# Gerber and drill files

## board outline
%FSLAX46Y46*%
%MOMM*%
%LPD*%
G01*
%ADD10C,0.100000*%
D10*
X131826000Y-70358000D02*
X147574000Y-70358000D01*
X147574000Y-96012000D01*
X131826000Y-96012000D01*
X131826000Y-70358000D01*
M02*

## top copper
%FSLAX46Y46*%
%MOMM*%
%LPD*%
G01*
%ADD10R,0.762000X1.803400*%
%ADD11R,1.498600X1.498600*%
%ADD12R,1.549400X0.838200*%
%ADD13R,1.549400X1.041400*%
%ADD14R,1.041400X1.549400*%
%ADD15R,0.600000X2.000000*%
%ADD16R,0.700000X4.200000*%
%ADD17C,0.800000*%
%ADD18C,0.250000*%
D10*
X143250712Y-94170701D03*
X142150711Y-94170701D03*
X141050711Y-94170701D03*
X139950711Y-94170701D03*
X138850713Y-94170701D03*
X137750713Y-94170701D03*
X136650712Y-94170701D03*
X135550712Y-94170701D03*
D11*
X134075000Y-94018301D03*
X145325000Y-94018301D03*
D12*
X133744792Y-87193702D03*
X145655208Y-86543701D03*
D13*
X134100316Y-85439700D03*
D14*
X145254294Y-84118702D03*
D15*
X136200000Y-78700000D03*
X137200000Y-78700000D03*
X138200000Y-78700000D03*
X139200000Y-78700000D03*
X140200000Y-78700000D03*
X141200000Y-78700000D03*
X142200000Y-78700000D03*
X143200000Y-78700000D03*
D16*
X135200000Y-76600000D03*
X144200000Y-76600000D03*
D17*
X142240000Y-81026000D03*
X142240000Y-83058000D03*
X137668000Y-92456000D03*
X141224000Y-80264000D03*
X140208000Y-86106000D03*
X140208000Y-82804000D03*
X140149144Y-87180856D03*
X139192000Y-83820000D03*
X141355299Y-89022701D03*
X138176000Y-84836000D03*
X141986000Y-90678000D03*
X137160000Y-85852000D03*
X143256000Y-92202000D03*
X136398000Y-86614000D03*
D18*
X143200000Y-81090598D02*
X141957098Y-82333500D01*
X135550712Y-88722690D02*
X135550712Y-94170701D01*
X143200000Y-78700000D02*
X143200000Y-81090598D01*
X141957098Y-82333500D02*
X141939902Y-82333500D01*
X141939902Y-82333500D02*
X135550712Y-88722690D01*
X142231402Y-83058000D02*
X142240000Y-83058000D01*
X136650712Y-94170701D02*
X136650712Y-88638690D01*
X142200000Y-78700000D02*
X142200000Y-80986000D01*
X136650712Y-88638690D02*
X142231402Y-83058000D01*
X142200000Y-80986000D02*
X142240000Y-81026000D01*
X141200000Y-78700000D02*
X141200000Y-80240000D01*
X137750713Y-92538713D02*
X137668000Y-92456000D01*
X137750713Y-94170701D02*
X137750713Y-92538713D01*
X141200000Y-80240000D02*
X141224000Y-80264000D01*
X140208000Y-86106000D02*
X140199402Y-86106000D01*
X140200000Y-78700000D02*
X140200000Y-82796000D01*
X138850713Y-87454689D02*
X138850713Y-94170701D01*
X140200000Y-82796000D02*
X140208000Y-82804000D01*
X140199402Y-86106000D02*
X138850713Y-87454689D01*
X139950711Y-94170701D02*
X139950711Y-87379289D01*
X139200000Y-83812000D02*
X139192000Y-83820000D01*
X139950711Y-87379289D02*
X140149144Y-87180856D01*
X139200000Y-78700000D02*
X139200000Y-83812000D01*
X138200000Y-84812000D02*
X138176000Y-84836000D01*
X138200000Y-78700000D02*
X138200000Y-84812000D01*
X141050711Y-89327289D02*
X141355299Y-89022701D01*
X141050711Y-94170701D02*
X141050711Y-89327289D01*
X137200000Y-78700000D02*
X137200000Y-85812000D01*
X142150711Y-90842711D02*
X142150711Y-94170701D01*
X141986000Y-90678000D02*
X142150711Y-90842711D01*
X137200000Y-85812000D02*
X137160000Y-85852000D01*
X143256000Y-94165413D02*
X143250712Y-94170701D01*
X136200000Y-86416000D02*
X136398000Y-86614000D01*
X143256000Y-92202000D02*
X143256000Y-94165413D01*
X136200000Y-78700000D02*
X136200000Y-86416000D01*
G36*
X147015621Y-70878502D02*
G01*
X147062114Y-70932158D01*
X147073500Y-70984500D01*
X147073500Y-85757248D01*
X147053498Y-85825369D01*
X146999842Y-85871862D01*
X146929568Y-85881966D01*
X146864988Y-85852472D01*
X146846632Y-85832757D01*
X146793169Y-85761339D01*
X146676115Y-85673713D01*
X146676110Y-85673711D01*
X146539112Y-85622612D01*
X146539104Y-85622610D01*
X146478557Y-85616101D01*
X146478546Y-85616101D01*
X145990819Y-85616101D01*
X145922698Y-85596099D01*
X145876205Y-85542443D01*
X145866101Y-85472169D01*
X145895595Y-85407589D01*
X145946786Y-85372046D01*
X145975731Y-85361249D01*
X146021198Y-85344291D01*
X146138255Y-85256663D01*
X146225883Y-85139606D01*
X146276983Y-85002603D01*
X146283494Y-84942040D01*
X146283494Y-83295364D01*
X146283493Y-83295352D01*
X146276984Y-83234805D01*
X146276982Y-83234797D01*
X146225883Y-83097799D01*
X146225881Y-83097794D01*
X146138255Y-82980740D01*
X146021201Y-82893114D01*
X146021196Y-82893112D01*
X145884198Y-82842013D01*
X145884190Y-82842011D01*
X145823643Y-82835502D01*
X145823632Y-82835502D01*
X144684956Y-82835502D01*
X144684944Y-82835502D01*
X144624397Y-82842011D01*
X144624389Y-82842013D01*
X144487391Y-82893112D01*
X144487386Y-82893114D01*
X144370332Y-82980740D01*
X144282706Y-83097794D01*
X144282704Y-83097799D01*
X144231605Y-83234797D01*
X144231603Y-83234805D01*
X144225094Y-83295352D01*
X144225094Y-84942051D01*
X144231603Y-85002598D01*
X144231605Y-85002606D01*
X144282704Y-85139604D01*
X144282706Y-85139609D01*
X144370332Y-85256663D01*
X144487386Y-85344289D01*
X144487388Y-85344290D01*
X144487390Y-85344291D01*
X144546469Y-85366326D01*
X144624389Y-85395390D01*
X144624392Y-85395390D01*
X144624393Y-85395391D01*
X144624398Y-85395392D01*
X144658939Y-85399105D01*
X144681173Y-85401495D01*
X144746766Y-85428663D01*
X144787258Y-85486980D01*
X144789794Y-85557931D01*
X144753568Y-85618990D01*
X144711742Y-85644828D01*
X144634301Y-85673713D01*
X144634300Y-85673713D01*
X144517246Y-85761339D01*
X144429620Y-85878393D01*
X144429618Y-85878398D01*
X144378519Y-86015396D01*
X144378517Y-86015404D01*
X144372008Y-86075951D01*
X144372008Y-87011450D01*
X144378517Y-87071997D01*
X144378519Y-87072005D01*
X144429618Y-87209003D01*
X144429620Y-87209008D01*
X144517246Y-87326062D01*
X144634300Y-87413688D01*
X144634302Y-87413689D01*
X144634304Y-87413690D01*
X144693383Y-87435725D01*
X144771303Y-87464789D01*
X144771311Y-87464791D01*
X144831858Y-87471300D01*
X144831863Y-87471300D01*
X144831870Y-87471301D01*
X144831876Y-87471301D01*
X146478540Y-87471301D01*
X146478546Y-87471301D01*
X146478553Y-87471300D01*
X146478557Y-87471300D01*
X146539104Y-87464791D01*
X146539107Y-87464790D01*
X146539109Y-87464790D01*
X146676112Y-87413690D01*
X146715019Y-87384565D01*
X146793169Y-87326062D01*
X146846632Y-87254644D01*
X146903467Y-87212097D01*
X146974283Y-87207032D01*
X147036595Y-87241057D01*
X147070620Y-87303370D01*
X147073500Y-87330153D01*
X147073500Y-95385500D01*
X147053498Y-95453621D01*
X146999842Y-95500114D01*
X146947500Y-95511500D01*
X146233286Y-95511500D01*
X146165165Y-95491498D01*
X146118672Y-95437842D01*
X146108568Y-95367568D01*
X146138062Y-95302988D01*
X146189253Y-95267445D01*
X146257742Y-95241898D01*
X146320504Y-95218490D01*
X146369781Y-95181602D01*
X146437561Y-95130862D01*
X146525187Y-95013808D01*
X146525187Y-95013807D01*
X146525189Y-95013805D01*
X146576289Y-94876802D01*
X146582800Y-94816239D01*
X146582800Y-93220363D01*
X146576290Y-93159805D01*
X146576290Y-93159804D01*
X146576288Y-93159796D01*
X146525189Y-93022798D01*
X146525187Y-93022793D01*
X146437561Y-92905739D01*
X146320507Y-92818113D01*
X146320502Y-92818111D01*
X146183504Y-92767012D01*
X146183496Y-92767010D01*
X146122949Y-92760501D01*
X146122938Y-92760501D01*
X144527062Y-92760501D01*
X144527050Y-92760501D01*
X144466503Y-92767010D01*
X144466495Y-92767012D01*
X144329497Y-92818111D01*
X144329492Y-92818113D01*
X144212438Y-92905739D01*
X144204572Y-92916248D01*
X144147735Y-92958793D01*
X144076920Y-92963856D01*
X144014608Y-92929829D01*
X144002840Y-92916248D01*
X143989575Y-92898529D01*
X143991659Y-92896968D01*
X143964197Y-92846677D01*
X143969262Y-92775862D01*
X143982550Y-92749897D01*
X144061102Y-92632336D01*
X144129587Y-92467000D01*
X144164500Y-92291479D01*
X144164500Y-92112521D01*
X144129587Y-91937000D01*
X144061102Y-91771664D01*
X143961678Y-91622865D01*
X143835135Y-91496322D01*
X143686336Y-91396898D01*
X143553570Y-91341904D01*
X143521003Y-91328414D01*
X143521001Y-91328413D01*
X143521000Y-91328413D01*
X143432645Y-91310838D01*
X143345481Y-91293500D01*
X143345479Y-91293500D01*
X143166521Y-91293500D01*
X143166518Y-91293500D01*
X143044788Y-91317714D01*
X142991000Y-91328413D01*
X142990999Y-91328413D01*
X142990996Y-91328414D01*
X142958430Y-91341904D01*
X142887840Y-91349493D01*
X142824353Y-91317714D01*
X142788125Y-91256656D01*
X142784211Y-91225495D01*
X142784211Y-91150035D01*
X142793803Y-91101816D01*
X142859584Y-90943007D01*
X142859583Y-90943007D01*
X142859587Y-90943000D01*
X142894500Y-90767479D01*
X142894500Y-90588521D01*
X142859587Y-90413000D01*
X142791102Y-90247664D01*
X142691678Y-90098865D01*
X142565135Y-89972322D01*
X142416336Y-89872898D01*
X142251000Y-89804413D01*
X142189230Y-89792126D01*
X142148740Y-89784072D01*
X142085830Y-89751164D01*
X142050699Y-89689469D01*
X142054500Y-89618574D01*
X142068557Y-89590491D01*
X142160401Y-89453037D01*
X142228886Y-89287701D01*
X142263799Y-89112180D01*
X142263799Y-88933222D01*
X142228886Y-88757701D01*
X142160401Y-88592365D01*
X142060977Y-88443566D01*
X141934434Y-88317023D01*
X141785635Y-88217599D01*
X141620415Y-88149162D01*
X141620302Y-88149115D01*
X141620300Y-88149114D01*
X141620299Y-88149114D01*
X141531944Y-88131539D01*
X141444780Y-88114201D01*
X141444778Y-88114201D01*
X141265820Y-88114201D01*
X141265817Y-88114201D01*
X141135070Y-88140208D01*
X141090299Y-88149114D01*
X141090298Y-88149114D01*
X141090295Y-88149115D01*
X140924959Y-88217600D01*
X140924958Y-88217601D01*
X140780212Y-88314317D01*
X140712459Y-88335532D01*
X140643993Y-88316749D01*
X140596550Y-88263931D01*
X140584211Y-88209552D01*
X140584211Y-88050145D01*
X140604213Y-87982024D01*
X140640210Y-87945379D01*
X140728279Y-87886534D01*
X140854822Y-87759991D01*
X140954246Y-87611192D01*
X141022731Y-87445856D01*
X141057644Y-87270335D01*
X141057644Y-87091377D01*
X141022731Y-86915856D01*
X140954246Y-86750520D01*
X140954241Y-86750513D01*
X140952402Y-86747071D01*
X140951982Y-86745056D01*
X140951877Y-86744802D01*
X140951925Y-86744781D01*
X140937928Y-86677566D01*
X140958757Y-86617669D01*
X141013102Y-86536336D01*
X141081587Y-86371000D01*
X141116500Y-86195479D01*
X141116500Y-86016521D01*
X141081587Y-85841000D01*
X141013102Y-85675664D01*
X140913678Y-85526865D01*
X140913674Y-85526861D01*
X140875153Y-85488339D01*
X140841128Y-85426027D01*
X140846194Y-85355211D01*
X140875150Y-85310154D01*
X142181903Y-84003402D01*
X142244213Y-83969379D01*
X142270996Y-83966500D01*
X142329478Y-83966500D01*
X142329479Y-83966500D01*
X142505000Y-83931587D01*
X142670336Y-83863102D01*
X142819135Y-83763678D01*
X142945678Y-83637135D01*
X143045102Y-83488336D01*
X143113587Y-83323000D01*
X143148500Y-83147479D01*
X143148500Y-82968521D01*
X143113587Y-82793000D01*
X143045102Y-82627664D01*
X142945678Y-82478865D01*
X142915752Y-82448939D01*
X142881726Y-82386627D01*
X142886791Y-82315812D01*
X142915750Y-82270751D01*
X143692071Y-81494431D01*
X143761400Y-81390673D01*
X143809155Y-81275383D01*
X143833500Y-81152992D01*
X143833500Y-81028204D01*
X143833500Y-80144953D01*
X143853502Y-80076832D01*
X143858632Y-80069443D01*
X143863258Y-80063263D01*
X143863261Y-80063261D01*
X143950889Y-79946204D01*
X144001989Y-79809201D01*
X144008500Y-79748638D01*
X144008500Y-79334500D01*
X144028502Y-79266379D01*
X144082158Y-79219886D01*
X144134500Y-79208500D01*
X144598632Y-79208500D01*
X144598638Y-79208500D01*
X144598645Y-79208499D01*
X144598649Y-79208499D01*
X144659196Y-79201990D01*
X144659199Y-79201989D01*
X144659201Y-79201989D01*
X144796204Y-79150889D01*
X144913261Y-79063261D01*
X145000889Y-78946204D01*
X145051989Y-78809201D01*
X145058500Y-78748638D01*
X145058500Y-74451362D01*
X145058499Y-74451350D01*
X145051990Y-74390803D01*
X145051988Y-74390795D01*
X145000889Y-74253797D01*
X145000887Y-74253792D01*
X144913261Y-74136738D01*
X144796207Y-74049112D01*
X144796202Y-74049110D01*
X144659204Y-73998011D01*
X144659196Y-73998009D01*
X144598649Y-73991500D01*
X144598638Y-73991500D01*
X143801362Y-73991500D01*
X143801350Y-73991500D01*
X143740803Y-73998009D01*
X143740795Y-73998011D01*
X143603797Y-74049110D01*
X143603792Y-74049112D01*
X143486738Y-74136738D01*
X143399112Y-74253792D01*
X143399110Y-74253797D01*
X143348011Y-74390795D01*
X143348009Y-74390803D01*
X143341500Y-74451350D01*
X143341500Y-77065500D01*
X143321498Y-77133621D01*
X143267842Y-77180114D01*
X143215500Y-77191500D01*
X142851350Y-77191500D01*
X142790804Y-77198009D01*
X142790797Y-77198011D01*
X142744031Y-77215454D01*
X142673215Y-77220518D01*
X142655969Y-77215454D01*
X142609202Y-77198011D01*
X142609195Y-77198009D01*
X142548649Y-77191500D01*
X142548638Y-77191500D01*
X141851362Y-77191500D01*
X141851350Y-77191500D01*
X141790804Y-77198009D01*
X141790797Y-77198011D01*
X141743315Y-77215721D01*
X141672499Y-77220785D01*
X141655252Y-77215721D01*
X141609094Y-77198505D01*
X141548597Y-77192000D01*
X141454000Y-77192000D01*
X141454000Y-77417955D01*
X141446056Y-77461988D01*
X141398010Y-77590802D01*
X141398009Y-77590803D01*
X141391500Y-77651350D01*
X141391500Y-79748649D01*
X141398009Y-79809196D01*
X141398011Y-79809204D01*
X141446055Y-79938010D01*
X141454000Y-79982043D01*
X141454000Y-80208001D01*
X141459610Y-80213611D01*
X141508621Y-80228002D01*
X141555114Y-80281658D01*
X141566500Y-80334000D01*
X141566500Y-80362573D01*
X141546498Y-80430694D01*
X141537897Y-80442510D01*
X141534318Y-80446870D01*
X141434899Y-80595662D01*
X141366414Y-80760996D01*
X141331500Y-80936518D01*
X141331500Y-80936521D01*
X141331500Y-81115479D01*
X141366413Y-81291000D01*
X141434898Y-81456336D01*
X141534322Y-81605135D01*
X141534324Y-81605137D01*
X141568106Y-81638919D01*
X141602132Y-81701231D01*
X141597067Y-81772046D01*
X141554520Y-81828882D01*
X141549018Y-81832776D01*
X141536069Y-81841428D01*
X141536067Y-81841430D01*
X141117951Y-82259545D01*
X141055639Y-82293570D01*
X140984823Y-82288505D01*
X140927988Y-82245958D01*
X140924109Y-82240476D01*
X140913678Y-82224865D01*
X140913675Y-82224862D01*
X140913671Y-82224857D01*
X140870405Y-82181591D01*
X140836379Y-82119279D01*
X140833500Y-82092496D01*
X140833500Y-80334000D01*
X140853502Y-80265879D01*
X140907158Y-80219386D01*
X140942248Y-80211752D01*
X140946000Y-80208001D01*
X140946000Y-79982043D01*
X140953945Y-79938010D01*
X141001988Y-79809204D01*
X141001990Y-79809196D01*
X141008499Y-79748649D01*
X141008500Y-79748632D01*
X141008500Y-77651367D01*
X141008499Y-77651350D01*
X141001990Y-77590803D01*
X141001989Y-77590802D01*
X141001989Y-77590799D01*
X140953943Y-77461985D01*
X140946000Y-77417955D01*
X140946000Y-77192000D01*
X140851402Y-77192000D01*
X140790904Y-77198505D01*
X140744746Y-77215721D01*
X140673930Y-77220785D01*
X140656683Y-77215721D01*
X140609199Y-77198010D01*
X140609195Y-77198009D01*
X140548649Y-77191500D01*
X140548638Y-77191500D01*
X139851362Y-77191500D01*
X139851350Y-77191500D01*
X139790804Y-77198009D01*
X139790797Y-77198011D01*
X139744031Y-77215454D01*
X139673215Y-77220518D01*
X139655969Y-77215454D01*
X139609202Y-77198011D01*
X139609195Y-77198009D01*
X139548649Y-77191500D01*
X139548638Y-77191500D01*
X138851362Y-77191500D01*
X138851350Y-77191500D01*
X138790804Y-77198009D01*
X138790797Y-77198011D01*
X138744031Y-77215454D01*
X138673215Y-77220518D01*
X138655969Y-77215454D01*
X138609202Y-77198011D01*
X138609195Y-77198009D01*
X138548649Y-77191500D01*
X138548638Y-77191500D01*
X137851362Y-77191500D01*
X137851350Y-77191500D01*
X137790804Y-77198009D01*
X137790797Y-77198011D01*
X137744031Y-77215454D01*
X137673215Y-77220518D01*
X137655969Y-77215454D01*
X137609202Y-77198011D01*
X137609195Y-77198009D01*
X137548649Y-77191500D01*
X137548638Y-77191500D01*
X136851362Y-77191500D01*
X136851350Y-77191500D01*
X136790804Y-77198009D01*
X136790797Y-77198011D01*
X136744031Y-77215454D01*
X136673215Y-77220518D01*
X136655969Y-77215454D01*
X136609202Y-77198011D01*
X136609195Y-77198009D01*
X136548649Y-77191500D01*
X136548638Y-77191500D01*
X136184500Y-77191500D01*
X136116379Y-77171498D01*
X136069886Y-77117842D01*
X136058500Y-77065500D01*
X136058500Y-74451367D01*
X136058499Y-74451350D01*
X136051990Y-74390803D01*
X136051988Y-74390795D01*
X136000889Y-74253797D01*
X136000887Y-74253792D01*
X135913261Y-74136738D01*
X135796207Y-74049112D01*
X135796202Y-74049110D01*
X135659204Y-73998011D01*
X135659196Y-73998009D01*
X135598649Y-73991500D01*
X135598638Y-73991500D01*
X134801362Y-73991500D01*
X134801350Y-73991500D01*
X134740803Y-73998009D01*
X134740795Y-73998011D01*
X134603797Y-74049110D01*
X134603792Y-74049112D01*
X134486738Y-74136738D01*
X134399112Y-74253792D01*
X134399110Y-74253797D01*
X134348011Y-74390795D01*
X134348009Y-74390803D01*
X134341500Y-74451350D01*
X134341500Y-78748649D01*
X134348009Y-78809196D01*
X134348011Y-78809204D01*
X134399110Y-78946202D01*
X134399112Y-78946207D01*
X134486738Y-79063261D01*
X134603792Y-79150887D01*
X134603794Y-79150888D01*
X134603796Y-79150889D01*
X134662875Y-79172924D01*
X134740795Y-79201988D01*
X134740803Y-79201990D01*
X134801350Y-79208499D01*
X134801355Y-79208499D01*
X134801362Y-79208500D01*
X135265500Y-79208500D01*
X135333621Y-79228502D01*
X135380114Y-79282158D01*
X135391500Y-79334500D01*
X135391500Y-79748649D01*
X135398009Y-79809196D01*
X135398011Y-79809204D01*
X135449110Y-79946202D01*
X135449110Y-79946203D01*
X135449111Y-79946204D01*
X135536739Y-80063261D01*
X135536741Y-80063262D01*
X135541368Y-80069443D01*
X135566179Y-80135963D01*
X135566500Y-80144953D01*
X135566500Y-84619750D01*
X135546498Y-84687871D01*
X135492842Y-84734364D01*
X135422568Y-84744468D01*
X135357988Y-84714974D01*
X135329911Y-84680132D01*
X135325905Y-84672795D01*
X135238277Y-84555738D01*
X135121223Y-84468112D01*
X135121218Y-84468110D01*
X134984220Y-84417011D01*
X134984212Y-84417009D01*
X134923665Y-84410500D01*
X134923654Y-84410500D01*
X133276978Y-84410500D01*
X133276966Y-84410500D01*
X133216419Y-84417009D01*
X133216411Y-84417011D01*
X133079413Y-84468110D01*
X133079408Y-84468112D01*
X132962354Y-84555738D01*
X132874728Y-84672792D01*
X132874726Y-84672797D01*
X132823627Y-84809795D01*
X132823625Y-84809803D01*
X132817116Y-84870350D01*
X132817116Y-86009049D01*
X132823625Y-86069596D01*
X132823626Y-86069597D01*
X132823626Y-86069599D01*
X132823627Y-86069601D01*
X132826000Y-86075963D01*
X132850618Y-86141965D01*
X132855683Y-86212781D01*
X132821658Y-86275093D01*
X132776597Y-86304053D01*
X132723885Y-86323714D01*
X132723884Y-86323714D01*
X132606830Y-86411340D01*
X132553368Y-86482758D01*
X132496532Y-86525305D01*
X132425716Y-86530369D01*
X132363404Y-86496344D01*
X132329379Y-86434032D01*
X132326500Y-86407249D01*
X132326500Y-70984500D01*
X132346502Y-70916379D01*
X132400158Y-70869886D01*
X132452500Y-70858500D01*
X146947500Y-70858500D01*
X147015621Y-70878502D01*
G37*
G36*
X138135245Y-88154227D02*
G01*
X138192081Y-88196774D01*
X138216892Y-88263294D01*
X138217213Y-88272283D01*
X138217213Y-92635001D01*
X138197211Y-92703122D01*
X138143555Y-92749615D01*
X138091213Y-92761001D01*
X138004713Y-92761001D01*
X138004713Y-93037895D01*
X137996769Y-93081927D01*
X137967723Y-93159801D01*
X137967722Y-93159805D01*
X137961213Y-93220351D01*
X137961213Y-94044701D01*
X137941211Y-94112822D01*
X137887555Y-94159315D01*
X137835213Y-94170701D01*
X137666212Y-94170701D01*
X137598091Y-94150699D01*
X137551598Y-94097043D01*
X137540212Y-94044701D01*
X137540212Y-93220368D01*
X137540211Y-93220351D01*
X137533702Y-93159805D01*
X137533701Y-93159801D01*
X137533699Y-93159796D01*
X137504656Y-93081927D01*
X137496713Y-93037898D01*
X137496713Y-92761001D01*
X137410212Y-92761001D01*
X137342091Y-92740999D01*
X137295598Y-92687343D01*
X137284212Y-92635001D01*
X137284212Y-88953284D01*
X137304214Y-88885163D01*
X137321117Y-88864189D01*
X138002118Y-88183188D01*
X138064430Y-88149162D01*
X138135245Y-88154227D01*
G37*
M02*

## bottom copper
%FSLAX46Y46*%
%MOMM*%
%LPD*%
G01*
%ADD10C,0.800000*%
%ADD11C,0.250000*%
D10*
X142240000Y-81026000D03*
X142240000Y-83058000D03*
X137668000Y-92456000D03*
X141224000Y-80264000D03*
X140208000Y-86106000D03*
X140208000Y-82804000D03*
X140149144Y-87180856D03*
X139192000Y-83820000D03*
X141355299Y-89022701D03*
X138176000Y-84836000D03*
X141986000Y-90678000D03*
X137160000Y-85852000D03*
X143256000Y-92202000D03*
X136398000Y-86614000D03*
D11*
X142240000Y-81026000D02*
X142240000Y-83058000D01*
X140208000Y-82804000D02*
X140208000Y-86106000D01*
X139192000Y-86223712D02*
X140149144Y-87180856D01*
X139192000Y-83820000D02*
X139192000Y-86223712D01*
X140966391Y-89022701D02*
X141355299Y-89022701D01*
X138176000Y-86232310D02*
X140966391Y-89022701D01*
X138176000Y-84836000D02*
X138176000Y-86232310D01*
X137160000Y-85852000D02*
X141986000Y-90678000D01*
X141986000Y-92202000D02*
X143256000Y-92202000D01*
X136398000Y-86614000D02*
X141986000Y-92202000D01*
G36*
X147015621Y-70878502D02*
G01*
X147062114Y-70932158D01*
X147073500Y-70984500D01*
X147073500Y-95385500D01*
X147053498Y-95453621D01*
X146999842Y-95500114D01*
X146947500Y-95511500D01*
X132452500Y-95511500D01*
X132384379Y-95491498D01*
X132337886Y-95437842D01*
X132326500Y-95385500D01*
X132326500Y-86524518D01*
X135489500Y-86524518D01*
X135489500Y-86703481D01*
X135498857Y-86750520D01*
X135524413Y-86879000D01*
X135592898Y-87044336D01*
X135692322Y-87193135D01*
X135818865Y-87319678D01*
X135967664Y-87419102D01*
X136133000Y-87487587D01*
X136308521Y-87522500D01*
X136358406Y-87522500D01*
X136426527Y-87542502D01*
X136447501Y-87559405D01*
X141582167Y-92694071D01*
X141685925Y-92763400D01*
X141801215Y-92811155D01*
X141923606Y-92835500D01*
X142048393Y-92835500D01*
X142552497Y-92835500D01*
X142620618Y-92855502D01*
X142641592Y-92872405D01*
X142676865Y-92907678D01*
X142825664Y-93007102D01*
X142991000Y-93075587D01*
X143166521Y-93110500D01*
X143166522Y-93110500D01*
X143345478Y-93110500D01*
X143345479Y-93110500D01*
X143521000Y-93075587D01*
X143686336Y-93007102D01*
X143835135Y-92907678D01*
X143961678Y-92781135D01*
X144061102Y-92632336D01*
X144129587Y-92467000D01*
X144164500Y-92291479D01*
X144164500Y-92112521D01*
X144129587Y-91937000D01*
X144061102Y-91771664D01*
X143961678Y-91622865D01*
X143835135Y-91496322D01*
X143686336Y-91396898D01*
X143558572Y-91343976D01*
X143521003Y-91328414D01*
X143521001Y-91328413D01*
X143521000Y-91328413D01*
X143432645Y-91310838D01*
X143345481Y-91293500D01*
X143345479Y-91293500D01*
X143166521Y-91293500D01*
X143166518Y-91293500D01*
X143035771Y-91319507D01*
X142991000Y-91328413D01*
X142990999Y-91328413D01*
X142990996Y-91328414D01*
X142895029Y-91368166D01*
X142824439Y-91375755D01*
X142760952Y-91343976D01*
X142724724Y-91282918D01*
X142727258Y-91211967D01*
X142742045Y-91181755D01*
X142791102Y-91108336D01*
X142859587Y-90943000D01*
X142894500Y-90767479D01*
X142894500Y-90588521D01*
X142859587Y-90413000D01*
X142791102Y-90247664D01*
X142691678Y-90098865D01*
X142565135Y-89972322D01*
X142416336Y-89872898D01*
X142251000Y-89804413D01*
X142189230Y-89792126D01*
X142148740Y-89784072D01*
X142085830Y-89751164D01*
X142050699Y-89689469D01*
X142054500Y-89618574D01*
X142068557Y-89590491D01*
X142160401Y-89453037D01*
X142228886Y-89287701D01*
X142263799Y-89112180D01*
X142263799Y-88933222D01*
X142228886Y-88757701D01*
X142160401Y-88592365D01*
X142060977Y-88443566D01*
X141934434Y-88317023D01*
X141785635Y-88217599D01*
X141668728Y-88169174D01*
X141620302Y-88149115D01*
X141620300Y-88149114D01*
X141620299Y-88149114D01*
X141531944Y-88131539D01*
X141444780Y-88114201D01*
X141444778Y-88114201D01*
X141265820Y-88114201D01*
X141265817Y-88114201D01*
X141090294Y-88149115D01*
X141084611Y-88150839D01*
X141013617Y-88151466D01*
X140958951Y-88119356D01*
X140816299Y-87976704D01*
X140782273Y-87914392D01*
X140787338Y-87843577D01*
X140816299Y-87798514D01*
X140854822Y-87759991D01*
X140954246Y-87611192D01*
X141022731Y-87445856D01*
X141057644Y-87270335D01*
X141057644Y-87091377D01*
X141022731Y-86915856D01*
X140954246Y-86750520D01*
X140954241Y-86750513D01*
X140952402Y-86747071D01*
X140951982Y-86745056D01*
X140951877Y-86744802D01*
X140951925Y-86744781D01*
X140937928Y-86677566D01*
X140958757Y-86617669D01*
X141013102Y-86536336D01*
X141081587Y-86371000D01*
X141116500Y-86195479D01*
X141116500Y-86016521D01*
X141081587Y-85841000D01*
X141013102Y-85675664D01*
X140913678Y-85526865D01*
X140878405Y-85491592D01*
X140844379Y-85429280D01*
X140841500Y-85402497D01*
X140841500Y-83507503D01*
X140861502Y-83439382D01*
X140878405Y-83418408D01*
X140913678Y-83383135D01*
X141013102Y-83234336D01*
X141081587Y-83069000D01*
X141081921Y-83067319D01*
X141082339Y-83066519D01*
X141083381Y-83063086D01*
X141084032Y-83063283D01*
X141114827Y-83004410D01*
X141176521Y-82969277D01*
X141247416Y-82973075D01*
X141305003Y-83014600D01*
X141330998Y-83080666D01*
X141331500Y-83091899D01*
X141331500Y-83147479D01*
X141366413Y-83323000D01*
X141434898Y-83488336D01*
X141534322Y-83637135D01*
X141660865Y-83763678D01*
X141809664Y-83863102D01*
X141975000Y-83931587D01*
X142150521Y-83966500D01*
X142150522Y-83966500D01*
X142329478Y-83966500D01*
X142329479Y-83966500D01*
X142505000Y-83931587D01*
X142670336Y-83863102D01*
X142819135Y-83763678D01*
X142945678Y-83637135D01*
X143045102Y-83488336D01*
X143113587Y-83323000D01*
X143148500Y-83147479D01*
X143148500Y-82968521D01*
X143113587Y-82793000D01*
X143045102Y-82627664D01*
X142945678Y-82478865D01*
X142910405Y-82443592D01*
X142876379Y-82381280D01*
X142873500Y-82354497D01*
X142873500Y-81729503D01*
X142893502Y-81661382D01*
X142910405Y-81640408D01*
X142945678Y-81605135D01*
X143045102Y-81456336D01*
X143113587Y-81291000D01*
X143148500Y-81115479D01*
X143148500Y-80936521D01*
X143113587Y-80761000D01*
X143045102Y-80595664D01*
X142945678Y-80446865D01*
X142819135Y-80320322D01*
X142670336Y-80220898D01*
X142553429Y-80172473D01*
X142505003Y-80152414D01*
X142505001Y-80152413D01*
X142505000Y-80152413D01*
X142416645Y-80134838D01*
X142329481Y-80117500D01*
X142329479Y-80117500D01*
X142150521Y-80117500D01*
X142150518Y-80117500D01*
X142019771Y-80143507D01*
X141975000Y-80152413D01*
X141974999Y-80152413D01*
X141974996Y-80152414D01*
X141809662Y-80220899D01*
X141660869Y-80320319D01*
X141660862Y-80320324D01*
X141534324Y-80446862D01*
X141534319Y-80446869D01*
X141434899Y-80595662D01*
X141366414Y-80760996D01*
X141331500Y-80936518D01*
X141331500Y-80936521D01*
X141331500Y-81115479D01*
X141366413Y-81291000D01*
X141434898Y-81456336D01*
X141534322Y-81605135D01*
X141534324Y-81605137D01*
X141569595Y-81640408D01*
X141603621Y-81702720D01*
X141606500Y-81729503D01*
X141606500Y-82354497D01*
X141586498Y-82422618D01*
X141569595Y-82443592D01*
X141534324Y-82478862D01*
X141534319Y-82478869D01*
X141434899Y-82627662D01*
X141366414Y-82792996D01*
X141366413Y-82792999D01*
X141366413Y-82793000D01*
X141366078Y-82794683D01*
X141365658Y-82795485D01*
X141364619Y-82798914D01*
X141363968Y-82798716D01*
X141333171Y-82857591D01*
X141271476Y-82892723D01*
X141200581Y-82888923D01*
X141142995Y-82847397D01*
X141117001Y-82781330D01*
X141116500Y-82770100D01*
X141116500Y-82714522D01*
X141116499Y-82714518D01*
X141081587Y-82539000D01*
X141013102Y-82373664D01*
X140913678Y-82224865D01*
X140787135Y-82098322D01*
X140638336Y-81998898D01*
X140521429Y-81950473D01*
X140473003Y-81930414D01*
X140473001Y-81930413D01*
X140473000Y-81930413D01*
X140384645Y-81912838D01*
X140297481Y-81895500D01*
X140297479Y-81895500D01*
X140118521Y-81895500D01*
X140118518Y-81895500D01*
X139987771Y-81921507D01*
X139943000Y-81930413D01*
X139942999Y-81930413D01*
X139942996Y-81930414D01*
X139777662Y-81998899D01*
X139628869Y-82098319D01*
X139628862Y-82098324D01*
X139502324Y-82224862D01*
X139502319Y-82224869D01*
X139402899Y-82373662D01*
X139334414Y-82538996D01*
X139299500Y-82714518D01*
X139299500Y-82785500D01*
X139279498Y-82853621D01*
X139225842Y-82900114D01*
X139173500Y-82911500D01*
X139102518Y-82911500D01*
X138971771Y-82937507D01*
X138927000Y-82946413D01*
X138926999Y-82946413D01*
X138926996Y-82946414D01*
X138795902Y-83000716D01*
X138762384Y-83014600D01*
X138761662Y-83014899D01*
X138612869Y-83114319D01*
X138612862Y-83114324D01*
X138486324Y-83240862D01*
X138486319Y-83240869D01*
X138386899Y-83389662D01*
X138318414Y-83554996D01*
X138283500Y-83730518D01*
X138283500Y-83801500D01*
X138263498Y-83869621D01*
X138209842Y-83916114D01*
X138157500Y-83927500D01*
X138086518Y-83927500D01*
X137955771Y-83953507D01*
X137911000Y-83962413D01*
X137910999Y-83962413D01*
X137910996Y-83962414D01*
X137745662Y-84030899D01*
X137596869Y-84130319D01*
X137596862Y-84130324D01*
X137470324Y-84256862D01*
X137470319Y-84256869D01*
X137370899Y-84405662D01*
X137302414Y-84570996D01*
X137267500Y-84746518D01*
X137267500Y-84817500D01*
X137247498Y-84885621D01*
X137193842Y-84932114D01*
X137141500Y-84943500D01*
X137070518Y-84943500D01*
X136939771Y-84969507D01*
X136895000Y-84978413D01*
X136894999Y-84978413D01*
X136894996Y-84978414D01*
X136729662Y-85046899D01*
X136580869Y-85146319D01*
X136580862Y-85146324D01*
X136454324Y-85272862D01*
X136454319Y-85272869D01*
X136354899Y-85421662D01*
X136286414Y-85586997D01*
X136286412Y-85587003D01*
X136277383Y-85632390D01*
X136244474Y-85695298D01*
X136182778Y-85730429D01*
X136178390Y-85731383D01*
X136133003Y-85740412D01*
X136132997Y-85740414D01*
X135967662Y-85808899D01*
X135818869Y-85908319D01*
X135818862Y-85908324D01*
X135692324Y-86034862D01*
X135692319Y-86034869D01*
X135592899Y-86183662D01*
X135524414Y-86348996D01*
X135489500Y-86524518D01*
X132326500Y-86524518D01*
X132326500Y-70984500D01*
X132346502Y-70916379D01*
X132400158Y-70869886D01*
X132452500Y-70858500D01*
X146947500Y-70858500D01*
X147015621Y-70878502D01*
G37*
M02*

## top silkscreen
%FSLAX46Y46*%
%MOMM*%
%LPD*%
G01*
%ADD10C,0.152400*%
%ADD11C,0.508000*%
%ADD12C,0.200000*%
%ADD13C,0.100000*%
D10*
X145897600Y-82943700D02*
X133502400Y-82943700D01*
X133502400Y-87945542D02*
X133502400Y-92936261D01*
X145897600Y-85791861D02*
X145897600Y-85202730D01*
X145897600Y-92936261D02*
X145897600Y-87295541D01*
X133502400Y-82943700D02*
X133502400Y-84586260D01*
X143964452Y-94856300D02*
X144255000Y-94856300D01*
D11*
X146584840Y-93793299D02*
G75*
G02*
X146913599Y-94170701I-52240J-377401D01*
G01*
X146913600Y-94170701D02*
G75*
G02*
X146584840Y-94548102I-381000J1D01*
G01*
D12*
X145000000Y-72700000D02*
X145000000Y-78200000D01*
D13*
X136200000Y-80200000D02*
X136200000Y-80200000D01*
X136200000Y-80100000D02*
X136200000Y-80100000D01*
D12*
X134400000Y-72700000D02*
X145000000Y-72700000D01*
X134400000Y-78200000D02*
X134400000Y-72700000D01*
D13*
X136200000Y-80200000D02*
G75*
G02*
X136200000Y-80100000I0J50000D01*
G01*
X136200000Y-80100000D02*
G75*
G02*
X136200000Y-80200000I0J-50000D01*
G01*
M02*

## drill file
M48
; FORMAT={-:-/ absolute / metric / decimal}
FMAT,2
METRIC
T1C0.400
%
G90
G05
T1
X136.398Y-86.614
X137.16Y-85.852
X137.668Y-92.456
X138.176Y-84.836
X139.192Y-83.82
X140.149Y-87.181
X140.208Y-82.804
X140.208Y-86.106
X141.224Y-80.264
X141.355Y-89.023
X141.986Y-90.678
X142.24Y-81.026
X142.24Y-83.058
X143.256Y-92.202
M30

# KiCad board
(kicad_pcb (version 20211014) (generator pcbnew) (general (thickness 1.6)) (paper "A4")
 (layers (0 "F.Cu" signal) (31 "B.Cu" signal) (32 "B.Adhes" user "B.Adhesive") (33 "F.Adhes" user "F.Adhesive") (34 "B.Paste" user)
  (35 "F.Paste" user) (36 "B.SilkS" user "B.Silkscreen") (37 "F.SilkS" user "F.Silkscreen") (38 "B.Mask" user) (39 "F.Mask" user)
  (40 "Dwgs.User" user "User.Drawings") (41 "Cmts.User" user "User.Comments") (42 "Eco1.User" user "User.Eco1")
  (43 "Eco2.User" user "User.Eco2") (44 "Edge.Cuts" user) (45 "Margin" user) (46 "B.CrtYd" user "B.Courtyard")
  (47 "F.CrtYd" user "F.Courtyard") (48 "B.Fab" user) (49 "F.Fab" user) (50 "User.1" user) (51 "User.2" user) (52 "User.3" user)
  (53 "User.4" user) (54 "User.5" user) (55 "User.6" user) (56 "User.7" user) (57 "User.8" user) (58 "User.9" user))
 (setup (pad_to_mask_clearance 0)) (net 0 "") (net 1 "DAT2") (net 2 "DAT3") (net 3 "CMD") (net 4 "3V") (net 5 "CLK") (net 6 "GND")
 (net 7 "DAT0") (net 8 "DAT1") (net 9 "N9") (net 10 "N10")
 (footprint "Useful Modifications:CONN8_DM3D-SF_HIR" (layer "F.Cu") (at 139.7 88.9)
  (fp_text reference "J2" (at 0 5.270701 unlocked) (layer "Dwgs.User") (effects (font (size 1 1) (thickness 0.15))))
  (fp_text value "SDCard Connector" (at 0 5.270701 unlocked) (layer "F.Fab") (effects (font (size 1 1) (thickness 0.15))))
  (fp_line (start 6.1976 -5.9563) (end -6.1976 -5.9563) (layer "F.SilkS") (width 0.1524))
  (fp_line (start -6.1976 -0.954458) (end -6.1976 4.036261) (layer "F.SilkS") (width 0.1524))
  (fp_line (start 6.1976 -3.108139) (end 6.1976 -3.69727) (layer "F.SilkS") (width 0.1524))
  (fp_line (start 6.1976 4.036261) (end 6.1976 -1.604459) (layer "F.SilkS") (width 0.1524))
  (fp_line (start -6.1976 -5.9563) (end -6.1976 -4.31374) (layer "F.SilkS") (width 0.1524))
  (fp_line (start 4.264452 5.9563) (end 4.555 5.9563) (layer "F.SilkS") (width 0.1524))
  (fp_arc (start 6.88484 4.893299) (mid 7.119884 5.020443) (end 7.2136 5.270701) (layer "F.SilkS") (width 0.508))
  (fp_arc (start 7.2136 5.270701) (mid 7.119884 5.520958) (end 6.88484 5.648102) (layer "F.SilkS") (width 0.508))
  (pad "1" smd rect (at 3.550712 5.270701) (size 0.762 1.8034) (layers "F.Cu" "F.Paste" "F.Mask") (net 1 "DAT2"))
  (pad "2" smd rect (at 2.450711 5.270701) (size 0.762 1.8034) (layers "F.Cu" "F.Paste" "F.Mask") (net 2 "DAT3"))
  (pad "3" smd rect (at 1.350711 5.270701) (size 0.762 1.8034) (layers "F.Cu" "F.Paste" "F.Mask") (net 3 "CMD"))
  (pad "4" smd rect (at 0.250711 5.270701) (size 0.762 1.8034) (layers "F.Cu" "F.Paste" "F.Mask") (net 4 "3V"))
  (pad "5" smd rect (at -0.849287 5.270701) (size 0.762 1.8034) (layers "F.Cu" "F.Paste" "F.Mask") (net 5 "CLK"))
  (pad "6" smd rect (at -1.949287 5.270701) (size 0.762 1.8034) (layers "F.Cu" "F.Paste" "F.Mask") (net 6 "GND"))
  (pad "7" smd rect (at -3.049288 5.270701) (size 0.762 1.8034) (layers "F.Cu" "F.Paste" "F.Mask") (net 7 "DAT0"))
  (pad "8" smd rect (at -4.149288 5.270701) (size 0.762 1.8034) (layers "F.Cu" "F.Paste" "F.Mask") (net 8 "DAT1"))
  (pad "9" smd rect (at -5.625 5.118301) (size 1.4986 1.4986) (layers "F.Cu" "F.Paste" "F.Mask"))
  (pad "10" smd rect (at 5.625 5.118301) (size 1.4986 1.4986) (layers "F.Cu" "F.Paste" "F.Mask"))
  (pad "11" smd rect (at -5.955208 -1.706298) (size 1.5494 0.8382) (layers "F.Cu" "F.Paste" "F.Mask"))
  (pad "12" smd rect (at 5.955208 -2.356299) (size 1.5494 0.8382) (layers "F.Cu" "F.Paste" "F.Mask"))
  (pad "13" smd rect (at -5.599684 -3.4603) (size 1.5494 1.0414) (layers "F.Cu" "F.Paste" "F.Mask"))
  (pad "14" smd rect (at 5.554294 -4.781298) (size 1.0414 1.5494) (layers "F.Cu" "F.Paste" "F.Mask")))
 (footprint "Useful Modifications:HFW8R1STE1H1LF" (layer "F.Cu") (at 139.7 76.2 180)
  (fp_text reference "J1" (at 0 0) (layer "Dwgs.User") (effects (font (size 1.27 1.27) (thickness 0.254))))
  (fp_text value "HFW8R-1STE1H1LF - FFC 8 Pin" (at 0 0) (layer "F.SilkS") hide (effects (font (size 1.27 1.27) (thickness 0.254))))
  (fp_line (start -5.3 3.5) (end -5.3 -2) (layer "F.SilkS") (width 0.2))
  (fp_line (start 3.5 -4) (end 3.5 -4) (layer "F.SilkS") (width 0.1))
  (fp_line (start 3.5 -3.9) (end 3.5 -3.9) (layer "F.SilkS") (width 0.1))
  (fp_line (start 5.3 3.5) (end -5.3 3.5) (layer "F.SilkS") (width 0.2))
  (fp_line (start 5.3 -2) (end 5.3 3.5) (layer "F.SilkS") (width 0.2))
  (fp_arc (start 3.5 -4) (mid 3.55 -3.95) (end 3.5 -3.9) (layer "F.SilkS") (width 0.1))
  (fp_arc (start 3.5 -3.9) (mid 3.45 -3.95) (end 3.5 -4) (layer "F.SilkS") (width 0.1))
  (pad "1" smd rect locked (at 3.5 -2.5 180) (size 0.6 2) (layers "F.Cu" "F.Paste" "F.Mask") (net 1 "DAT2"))
  (pad "2" smd rect locked (at 2.5 -2.5 180) (size 0.6 2) (layers "F.Cu" "F.Paste" "F.Mask") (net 2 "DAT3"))
  (pad "3" smd rect locked (at 1.5 -2.5 180) (size 0.6 2) (layers "F.Cu" "F.Paste" "F.Mask") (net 3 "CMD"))
  (pad "4" smd rect locked (at 0.5 -2.5 180) (size 0.6 2) (layers "F.Cu" "F.Paste" "F.Mask") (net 4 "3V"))
  (pad "5" smd rect locked (at -0.5 -2.5 180) (size 0.6 2) (layers "F.Cu" "F.Paste" "F.Mask") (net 5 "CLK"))
  (pad "6" smd rect locked (at -1.5 -2.5 180) (size 0.6 2) (layers "F.Cu" "F.Paste" "F.Mask") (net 6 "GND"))
  (pad "7" smd rect locked (at -2.5 -2.5 180) (size 0.6 2) (layers "F.Cu" "F.Paste" "F.Mask") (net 7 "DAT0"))
  (pad "8" smd rect locked (at -3.5 -2.5 180) (size 0.6 2) (layers "F.Cu" "F.Paste" "F.Mask") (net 8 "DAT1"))
  (pad "MP1" smd rect locked (at 4.5 -0.4 180) (size 0.7 4.2) (layers "F.Cu" "F.Paste" "F.Mask") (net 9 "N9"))
  (pad "MP2" smd rect locked (at -4.5 -0.4 180) (size 0.7 4.2) (layers "F.Cu" "F.Paste" "F.Mask") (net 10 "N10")))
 (gr_rect (start 131.826 70.358) (end 147.574 96.012) (layer "Edge.Cuts") (width 0.1) (fill none))
 (segment (start 143.2 81.090598) (end 141.957098 82.3335) (width 0.25) (layer "F.Cu") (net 8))
 (segment (start 135.550712 88.72269) (end 135.550712 94.170701) (width 0.25) (layer "F.Cu") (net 8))
 (segment (start 143.2 78.7) (end 143.2 81.090598) (width 0.25) (layer "F.Cu") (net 8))
 (segment (start 141.957098 82.3335) (end 141.939902 82.3335) (width 0.25) (layer "F.Cu") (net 8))
 (segment (start 141.939902 82.3335) (end 135.550712 88.72269) (width 0.25) (layer "F.Cu") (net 8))
 (segment (start 142.231402 83.058) (end 142.24 83.058) (width 0.25) (layer "F.Cu") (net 7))
 (segment (start 136.650712 94.170701) (end 136.650712 88.63869) (width 0.25) (layer "F.Cu") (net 7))
 (segment (start 142.2 78.7) (end 142.2 80.986) (width 0.25) (layer "F.Cu") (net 7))
 (segment (start 136.650712 88.63869) (end 142.231402 83.058) (width 0.25) (layer "F.Cu") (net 7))
 (segment (start 142.2 80.986) (end 142.24 81.026) (width 0.25) (layer "F.Cu") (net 7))
 (via (at 142.24 81.026) (size 0.8) (drill 0.4) (layers "F.Cu" "B.Cu") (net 7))
 (via (at 142.24 83.058) (size 0.8) (drill 0.4) (layers "F.Cu" "B.Cu") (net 7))
 (segment (start 142.24 81.026) (end 142.24 83.058) (width 0.25) (layer "B.Cu") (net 7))
 (segment (start 141.2 78.7) (end 141.2 80.24) (width 0.25) (layer "F.Cu") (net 6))
 (segment (start 137.750713 92.538713) (end 137.668 92.456) (width 0.25) (layer "F.Cu") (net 6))
 (segment (start 137.750713 94.170701) (end 137.750713 92.538713) (width 0.25) (layer "F.Cu") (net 6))
 (segment (start 141.2 80.24) (end 141.224 80.264) (width 0.25) (layer "F.Cu") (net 6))
 (via (at 137.668 92.456) (size 0.8) (drill 0.4) (layers "F.Cu" "B.Cu") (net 6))
 (via (at 141.224 80.264) (size 0.8) (drill 0.4) (layers "F.Cu" "B.Cu") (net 6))
 (segment (start 140.208 86.106) (end 140.199402 86.106) (width 0.25) (layer "F.Cu") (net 5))
 (segment (start 140.2 78.7) (end 140.2 82.796) (width 0.25) (layer "F.Cu") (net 5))
 (segment (start 138.850713 87.454689) (end 138.850713 94.170701) (width 0.25) (layer "F.Cu") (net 5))
 (segment (start 140.2 82.796) (end 140.208 82.804) (width 0.25) (layer "F.Cu") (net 5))
 (segment (start 140.199402 86.106) (end 138.850713 87.454689) (width 0.25) (layer "F.Cu") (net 5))
 (via (at 140.208 86.106) (size 0.8) (drill 0.4) (layers "F.Cu" "B.Cu") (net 5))
 (via (at 140.208 82.804) (size 0.8) (drill 0.4) (layers "F.Cu" "B.Cu") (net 5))
 (segment (start 140.208 82.804) (end 140.208 86.106) (width 0.25) (layer "B.Cu") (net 5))
 (segment (start 139.950711 94.170701) (end 139.950711 87.379289) (width 0.25) (layer "F.Cu") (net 4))
 (segment (start 139.2 83.812) (end 139.192 83.82) (width 0.25) (layer "F.Cu") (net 4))
 (segment (start 139.950711 87.379289) (end 140.149144 87.180856) (width 0.25) (layer "F.Cu") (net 4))
 (segment (start 139.2 78.7) (end 139.2 83.812) (width 0.25) (layer "F.Cu") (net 4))
 (via (at 140.149144 87.180856) (size 0.8) (drill 0.4) (layers "F.Cu" "B.Cu") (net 4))
 (via (at 139.192 83.82) (size 0.8) (drill 0.4) (layers "F.Cu" "B.Cu") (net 4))
 (segment (start 139.192 86.223712) (end 140.149144 87.180856) (width 0.25) (layer "B.Cu") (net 4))
 (segment (start 139.192 83.82) (end 139.192 86.223712) (width 0.25) (layer "B.Cu") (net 4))
 (segment (start 138.2 84.812) (end 138.176 84.836) (width 0.25) (layer "F.Cu") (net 3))
 (segment (start 138.2 78.7) (end 138.2 84.812) (width 0.25) (layer "F.Cu") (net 3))
 (segment (start 141.050711 89.327289) (end 141.355299 89.022701) (width 0.25) (layer "F.Cu") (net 3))
 (segment (start 141.050711 94.170701) (end 141.050711 89.327289) (width 0.25) (layer "F.Cu") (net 3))
 (via (at 141.355299 89.022701) (size 0.8) (drill 0.4) (layers "F.Cu" "B.Cu") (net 3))
 (via (at 138.176 84.836) (size 0.8) (drill 0.4) (layers "F.Cu" "B.Cu") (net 3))
 (segment (start 140.966391 89.022701) (end 141.355299 89.022701) (width 0.25) (layer "B.Cu") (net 3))
 (segment (start 138.176 86.23231) (end 140.966391 89.022701) (width 0.25) (layer "B.Cu") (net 3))
 (segment (start 138.176 84.836) (end 138.176 86.23231) (width 0.25) (layer "B.Cu") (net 3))
 (segment (start 137.2 78.7) (end 137.2 85.812) (width 0.25) (layer "F.Cu") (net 2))
 (segment (start 142.150711 90.842711) (end 142.150711 94.170701) (width 0.25) (layer "F.Cu") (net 2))
 (segment (start 141.986 90.678) (end 142.150711 90.842711) (width 0.25) (layer "F.Cu") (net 2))
 (segment (start 137.2 85.812) (end 137.16 85.852) (width 0.25) (layer "F.Cu") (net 2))
 (via (at 141.986 90.678) (size 0.8) (drill 0.4) (layers "F.Cu" "B.Cu") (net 2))
 (via (at 137.16 85.852) (size 0.8) (drill 0.4) (layers "F.Cu" "B.Cu") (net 2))
 (segment (start 137.16 85.852) (end 141.986 90.678) (width 0.25) (layer "B.Cu") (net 2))
 (segment (start 143.256 94.165413) (end 143.250712 94.170701) (width 0.25) (layer "F.Cu") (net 1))
 (segment (start 136.2 86.416) (end 136.398 86.614) (width 0.25) (layer "F.Cu") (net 1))
 (segment (start 143.256 92.202) (end 143.256 94.165413) (width 0.25) (layer "F.Cu") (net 1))
 (segment (start 136.2 78.7) (end 136.2 86.416) (width 0.25) (layer "F.Cu") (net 1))
 (via (at 143.256 92.202) (size 0.8) (drill 0.4) (layers "F.Cu" "B.Cu") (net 1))
 (via (at 136.398 86.614) (size 0.8) (drill 0.4) (layers "F.Cu" "B.Cu") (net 1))
 (segment (start 141.986 92.202) (end 143.256 92.202) (width 0.25) (layer "B.Cu") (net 1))
 (segment (start 136.398 86.614) (end 141.986 92.202) (width 0.25) (layer "B.Cu") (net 1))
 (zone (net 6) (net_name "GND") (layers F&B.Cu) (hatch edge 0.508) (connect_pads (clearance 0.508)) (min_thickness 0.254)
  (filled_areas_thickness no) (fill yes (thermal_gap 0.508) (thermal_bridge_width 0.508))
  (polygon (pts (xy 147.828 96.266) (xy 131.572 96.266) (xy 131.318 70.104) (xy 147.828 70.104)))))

